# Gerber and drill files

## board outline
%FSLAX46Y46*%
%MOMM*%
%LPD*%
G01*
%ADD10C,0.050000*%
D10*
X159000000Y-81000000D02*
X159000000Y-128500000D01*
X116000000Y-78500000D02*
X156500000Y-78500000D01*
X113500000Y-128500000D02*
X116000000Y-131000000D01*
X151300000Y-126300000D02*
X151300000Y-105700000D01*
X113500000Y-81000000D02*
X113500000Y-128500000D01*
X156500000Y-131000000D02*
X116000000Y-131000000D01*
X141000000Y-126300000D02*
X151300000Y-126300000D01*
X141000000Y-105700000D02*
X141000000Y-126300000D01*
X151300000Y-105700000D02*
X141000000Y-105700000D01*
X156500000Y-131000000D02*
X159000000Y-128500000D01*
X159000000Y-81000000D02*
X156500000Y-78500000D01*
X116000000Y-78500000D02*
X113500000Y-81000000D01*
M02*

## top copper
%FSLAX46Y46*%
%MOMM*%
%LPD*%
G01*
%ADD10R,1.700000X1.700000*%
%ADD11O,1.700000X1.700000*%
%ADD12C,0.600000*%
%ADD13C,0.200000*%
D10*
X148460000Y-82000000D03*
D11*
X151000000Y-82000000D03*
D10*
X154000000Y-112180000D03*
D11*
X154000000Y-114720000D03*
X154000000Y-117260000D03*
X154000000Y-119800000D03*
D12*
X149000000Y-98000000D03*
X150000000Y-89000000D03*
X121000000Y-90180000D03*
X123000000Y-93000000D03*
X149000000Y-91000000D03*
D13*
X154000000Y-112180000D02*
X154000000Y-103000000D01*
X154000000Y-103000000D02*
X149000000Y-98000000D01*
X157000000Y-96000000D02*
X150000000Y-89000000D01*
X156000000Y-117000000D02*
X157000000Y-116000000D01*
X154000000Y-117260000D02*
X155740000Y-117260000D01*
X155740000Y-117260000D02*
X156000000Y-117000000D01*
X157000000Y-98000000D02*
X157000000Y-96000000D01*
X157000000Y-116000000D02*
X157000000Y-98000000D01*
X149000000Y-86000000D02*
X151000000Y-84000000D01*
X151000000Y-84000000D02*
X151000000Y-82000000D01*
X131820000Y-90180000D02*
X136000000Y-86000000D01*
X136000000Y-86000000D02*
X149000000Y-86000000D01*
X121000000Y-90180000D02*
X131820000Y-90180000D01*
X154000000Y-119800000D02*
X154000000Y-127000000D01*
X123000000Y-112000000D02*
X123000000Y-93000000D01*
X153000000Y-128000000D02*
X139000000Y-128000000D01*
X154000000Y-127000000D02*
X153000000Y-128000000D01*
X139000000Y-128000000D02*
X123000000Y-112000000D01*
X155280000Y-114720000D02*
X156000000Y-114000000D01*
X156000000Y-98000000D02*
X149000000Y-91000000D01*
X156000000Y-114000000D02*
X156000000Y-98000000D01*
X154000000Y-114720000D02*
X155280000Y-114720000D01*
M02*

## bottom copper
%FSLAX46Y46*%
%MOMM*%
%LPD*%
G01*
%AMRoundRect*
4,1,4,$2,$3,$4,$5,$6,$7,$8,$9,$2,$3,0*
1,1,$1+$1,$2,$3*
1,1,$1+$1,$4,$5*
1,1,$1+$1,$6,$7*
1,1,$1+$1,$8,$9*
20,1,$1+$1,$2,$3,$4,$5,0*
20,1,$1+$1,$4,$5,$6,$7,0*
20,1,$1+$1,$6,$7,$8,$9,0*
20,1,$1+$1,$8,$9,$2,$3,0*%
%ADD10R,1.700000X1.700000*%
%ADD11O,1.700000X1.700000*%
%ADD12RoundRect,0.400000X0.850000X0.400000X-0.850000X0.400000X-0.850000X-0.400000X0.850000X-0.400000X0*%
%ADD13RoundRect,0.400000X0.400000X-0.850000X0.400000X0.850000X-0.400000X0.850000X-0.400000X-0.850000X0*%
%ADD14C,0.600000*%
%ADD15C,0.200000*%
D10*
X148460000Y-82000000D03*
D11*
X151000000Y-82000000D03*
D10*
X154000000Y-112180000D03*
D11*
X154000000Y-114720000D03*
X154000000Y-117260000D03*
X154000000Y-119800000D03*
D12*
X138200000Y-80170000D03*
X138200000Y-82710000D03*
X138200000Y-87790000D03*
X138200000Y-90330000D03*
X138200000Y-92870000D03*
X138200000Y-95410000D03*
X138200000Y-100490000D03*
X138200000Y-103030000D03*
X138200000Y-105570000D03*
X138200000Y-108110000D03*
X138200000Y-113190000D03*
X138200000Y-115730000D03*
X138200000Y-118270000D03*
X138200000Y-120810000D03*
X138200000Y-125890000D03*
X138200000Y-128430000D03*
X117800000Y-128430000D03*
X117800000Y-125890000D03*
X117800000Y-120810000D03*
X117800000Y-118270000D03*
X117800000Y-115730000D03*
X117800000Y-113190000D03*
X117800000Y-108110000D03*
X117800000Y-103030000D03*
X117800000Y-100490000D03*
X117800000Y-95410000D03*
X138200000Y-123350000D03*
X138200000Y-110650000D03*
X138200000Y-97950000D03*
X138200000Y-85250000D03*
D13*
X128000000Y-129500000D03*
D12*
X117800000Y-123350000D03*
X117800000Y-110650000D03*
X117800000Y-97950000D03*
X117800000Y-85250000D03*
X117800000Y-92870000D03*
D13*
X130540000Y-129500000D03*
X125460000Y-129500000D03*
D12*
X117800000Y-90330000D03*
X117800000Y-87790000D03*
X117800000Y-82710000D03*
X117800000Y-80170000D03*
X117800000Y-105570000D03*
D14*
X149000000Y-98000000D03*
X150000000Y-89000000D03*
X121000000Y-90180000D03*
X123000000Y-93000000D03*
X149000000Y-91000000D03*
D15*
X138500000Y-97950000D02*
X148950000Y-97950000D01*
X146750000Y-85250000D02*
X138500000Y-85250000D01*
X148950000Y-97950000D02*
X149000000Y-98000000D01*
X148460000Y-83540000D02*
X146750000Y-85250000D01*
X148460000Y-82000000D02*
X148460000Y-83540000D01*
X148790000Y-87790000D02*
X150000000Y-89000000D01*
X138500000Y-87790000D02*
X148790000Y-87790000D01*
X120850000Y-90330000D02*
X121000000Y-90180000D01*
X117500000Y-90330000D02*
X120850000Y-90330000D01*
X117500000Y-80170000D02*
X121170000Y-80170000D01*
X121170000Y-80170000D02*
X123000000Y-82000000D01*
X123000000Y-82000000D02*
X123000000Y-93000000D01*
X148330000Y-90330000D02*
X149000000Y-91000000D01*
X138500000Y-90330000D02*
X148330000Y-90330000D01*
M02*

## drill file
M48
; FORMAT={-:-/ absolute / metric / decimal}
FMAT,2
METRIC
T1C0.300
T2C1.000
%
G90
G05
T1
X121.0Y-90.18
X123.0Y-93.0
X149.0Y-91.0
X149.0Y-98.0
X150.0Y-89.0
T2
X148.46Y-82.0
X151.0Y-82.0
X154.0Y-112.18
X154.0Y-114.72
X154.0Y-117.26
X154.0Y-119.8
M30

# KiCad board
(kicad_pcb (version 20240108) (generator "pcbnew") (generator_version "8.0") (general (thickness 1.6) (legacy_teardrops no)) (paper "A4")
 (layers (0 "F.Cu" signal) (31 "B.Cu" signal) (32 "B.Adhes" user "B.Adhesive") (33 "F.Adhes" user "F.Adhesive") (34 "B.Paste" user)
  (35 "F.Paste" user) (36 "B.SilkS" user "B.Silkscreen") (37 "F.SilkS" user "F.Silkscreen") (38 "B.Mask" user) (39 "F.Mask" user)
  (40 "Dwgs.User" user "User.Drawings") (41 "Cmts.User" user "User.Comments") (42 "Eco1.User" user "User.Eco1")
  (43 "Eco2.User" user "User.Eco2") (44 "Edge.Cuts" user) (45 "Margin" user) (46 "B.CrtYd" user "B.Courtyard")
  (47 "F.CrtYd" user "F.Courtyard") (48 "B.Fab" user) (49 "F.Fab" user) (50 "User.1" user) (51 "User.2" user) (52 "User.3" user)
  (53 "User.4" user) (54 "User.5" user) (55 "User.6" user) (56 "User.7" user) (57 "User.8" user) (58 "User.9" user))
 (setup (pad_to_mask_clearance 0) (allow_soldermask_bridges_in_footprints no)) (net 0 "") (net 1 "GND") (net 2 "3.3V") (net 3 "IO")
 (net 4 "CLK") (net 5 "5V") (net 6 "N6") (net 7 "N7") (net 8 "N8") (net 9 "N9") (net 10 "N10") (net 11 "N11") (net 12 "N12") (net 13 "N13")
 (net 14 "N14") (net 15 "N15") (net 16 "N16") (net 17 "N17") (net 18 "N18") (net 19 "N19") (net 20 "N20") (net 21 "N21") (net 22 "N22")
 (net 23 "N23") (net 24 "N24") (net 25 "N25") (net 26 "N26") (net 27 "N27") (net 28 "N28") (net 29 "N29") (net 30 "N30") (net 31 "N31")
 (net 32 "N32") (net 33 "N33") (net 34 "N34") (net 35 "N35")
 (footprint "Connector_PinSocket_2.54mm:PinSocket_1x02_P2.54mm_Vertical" (layer "F.Cu") (at 148.46 82 90)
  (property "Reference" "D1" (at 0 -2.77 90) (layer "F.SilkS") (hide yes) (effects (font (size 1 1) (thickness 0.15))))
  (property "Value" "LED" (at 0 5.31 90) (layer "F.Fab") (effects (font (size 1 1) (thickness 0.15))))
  (pad "1" thru_hole rect (at 0 0 90) (size 1.7 1.7) (drill 1) (layers "*.Cu" "*.Mask") (remove_unused_layers no) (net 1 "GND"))
  (pad "2" thru_hole oval (at 0 2.54 90) (size 1.7 1.7) (drill 1) (layers "*.Cu" "*.Mask") (remove_unused_layers no) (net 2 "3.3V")))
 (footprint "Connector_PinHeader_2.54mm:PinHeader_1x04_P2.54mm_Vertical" (layer "F.Cu") (at 154 112.18)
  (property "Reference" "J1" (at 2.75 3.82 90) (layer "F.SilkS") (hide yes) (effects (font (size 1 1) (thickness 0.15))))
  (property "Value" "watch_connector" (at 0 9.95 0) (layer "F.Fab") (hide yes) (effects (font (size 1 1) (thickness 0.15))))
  (pad "1" thru_hole rect (at 0 0) (size 1.7 1.7) (drill 1) (layers "*.Cu" "*.Mask") (remove_unused_layers no) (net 1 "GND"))
  (pad "2" thru_hole oval (at 0 2.54) (size 1.7 1.7) (drill 1) (layers "*.Cu" "*.Mask") (remove_unused_layers no) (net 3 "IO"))
  (pad "3" thru_hole oval (at 0 5.08) (size 1.7 1.7) (drill 1) (layers "*.Cu" "*.Mask") (remove_unused_layers no) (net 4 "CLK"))
  (pad "4" thru_hole oval (at 0 7.62) (size 1.7 1.7) (drill 1) (layers "*.Cu" "*.Mask") (remove_unused_layers no) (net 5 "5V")))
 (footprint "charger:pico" (layer "B.Cu") (at 128 104.3 180)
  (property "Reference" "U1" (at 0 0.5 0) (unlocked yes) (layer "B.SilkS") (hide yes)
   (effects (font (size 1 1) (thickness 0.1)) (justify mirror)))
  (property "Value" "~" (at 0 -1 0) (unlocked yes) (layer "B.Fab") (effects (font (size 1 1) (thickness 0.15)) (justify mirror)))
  (pad "0" smd roundrect (at -10.5 24.13 180) (size 2.5 1.6) (drill (offset 0.3 0)) (layers "B.Cu" "B.Paste" "B.Mask")
   (roundrect_rratio 0.25) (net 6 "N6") (thermal_bridge_angle 45))
  (pad "1" smd roundrect (at -10.5 21.59 180) (size 2.5 1.6) (drill (offset 0.3 0)) (layers "B.Cu" "B.Paste" "B.Mask")
   (roundrect_rratio 0.25) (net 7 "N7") (thermal_bridge_angle 45))
  (pad "2" smd roundrect (at -10.5 16.51 180) (size 2.5 1.6) (drill (offset 0.3 0)) (layers "B.Cu" "B.Paste" "B.Mask")
   (roundrect_rratio 0.25) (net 4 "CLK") (thermal_bridge_angle 45))
  (pad "3" smd roundrect (at -10.5 13.97 180) (size 2.5 1.6) (drill (offset 0.3 0)) (layers "B.Cu" "B.Paste" "B.Mask")
   (roundrect_rratio 0.25) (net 3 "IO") (thermal_bridge_angle 45))
  (pad "4" smd roundrect (at -10.5 11.43 180) (size 2.5 1.6) (drill (offset 0.3 0)) (layers "B.Cu" "B.Paste" "B.Mask")
   (roundrect_rratio 0.25) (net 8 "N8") (thermal_bridge_angle 45))
  (pad "5" smd roundrect (at -10.5 8.89 180) (size 2.5 1.6) (drill (offset 0.3 0)) (layers "B.Cu" "B.Paste" "B.Mask")
   (roundrect_rratio 0.25) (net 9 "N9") (thermal_bridge_angle 45))
  (pad "6" smd roundrect (at -10.5 3.81 180) (size 2.5 1.6) (drill (offset 0.3 0)) (layers "B.Cu" "B.Paste" "B.Mask")
   (roundrect_rratio 0.25) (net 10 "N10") (thermal_bridge_angle 45))
  (pad "7" smd roundrect (at -10.5 1.27 180) (size 2.5 1.6) (drill (offset 0.3 0)) (layers "B.Cu" "B.Paste" "B.Mask")
   (roundrect_rratio 0.25) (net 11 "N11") (thermal_bridge_angle 45))
  (pad "8" smd roundrect (at -10.5 -1.27 180) (size 2.5 1.6) (drill (offset 0.3 0)) (layers "B.Cu" "B.Paste" "B.Mask")
   (roundrect_rratio 0.25) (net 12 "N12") (thermal_bridge_angle 45))
  (pad "9" smd roundrect (at -10.5 -3.81 180) (size 2.5 1.6) (drill (offset 0.3 0)) (layers "B.Cu" "B.Paste" "B.Mask")
   (roundrect_rratio 0.25) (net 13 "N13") (thermal_bridge_angle 45))
  (pad "10" smd roundrect (at -10.5 -8.89 180) (size 2.5 1.6) (drill (offset 0.3 0)) (layers "B.Cu" "B.Paste" "B.Mask")
   (roundrect_rratio 0.25) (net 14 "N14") (thermal_bridge_angle 45))
  (pad "11" smd roundrect (at -10.5 -11.43 180) (size 2.5 1.6) (drill (offset 0.3 0)) (layers "B.Cu" "B.Paste" "B.Mask")
   (roundrect_rratio 0.25) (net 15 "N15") (thermal_bridge_angle 45))
  (pad "12" smd roundrect (at -10.5 -13.97 180) (size 2.5 1.6) (drill (offset 0.3 0)) (layers "B.Cu" "B.Paste" "B.Mask")
   (roundrect_rratio 0.25) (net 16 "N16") (thermal_bridge_angle 45))
  (pad "13" smd roundrect (at -10.5 -16.51 180) (size 2.5 1.6) (drill (offset 0.3 0)) (layers "B.Cu" "B.Paste" "B.Mask")
   (roundrect_rratio 0.25) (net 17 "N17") (thermal_bridge_angle 45))
  (pad "14" smd roundrect (at -10.5 -21.59 180) (size 2.5 1.6) (drill (offset 0.3 0)) (layers "B.Cu" "B.Paste" "B.Mask")
   (roundrect_rratio 0.25) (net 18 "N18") (thermal_bridge_angle 45))
  (pad "15" smd roundrect (at -10.5 -24.13 180) (size 2.5 1.6) (drill (offset 0.3 0)) (layers "B.Cu" "B.Paste" "B.Mask")
   (roundrect_rratio 0.25) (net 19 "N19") (thermal_bridge_angle 45))
  (pad "16" smd roundrect (at 10.5 -24.13 180) (size 2.5 1.6) (drill (offset -0.3 0)) (layers "B.Cu" "B.Paste" "B.Mask")
   (roundrect_rratio 0.25) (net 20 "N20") (thermal_bridge_angle 45))
  (pad "17" smd roundrect (at 10.5 -21.59 180) (size 2.5 1.6) (drill (offset -0.3 0)) (layers "B.Cu" "B.Paste" "B.Mask")
   (roundrect_rratio 0.25) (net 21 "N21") (thermal_bridge_angle 45))
  (pad "18" smd roundrect (at 10.5 -16.51 180) (size 2.5 1.6) (drill (offset -0.3 0)) (layers "B.Cu" "B.Paste" "B.Mask")
   (roundrect_rratio 0.25) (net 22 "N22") (thermal_bridge_angle 45))
  (pad "19" smd roundrect (at 10.5 -13.97 180) (size 2.5 1.6) (drill (offset -0.3 0)) (layers "B.Cu" "B.Paste" "B.Mask")
   (roundrect_rratio 0.25) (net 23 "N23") (thermal_bridge_angle 45))
  (pad "20" smd roundrect (at 10.5 -11.43 180) (size 2.5 1.6) (drill (offset -0.3 0)) (layers "B.Cu" "B.Paste" "B.Mask")
   (roundrect_rratio 0.25) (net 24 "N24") (thermal_bridge_angle 45))
  (pad "21" smd roundrect (at 10.5 -8.89 180) (size 2.5 1.6) (drill (offset -0.3 0)) (layers "B.Cu" "B.Paste" "B.Mask")
   (roundrect_rratio 0.25) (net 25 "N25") (thermal_bridge_angle 45))
  (pad "22" smd roundrect (at 10.5 -3.81 180) (size 2.5 1.6) (drill (offset -0.3 0)) (layers "B.Cu" "B.Paste" "B.Mask")
   (roundrect_rratio 0.25) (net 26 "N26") (thermal_bridge_angle 45))
  (pad "26" smd roundrect (at 10.5 1.27 180) (size 2.5 1.6) (drill (offset -0.3 0)) (layers "B.Cu" "B.Paste" "B.Mask")
   (roundrect_rratio 0.25) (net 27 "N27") (thermal_bridge_angle 45))
  (pad "27" smd roundrect (at 10.5 3.81 180) (size 2.5 1.6) (drill (offset -0.3 0)) (layers "B.Cu" "B.Paste" "B.Mask")
   (roundrect_rratio 0.25) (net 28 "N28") (thermal_bridge_angle 45))
  (pad "28" smd roundrect (at 10.5 8.89 180) (size 2.5 1.6) (drill (offset -0.3 0)) (layers "B.Cu" "B.Paste" "B.Mask")
   (roundrect_rratio 0.25) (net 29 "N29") (thermal_bridge_angle 45))
  (pad "29" smd roundrect (at -10.5 -19.05 180) (size 2.5 1.6) (drill (offset 0.3 0)) (layers "B.Cu" "B.Paste" "B.Mask")
   (roundrect_rratio 0.25) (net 1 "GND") (thermal_bridge_angle 45))
  (pad "29" smd roundrect (at -10.5 -6.35 180) (size 2.5 1.6) (drill (offset 0.3 0)) (layers "B.Cu" "B.Paste" "B.Mask")
   (roundrect_rratio 0.25) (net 1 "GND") (thermal_bridge_angle 45))
  (pad "29" smd roundrect (at -10.5 6.35 180) (size 2.5 1.6) (drill (offset 0.3 0)) (layers "B.Cu" "B.Paste" "B.Mask")
   (roundrect_rratio 0.25) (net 1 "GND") (thermal_bridge_angle 45))
  (pad "29" smd roundrect (at -10.5 19.05 180) (size 2.5 1.6) (drill (offset 0.3 0)) (layers "B.Cu" "B.Paste" "B.Mask")
   (roundrect_rratio 0.25) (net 1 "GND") (thermal_bridge_angle 45))
  (pad "29" smd roundrect (at 0 -25.5 90) (size 2.5 1.6) (drill (offset 0.3 0)) (layers "B.Cu" "B.Paste" "B.Mask") (roundrect_rratio 0.25)
   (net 1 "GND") (thermal_bridge_angle 45))
  (pad "29" smd roundrect (at 10.5 -19.05 180) (size 2.5 1.6) (drill (offset -0.3 0)) (layers "B.Cu" "B.Paste" "B.Mask")
   (roundrect_rratio 0.25) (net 1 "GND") (thermal_bridge_angle 45))
  (pad "29" smd roundrect (at 10.5 -6.35 180) (size 2.5 1.6) (drill (offset -0.3 0)) (layers "B.Cu" "B.Paste" "B.Mask")
   (roundrect_rratio 0.25) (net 1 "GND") (thermal_bridge_angle 45))
  (pad "29" smd roundrect (at 10.5 6.35 180) (size 2.5 1.6) (drill (offset -0.3 0)) (layers "B.Cu" "B.Paste" "B.Mask")
   (roundrect_rratio 0.25) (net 1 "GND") (thermal_bridge_angle 45))
  (pad "29" smd roundrect (at 10.5 19.05 180) (size 2.5 1.6) (drill (offset -0.3 0)) (layers "B.Cu" "B.Paste" "B.Mask")
   (roundrect_rratio 0.25) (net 1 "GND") (thermal_bridge_angle 45))
  (pad "30" smd roundrect (at 10.5 11.43 180) (size 2.5 1.6) (drill (offset -0.3 0)) (layers "B.Cu" "B.Paste" "B.Mask")
   (roundrect_rratio 0.25) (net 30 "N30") (thermal_bridge_angle 45))
  (pad "31" smd roundrect (at -2.54 -25.5 90) (size 2.5 1.6) (drill (offset 0.3 0)) (layers "B.Cu" "B.Paste" "B.Mask")
   (roundrect_rratio 0.25) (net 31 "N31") (thermal_bridge_angle 45))
  (pad "32" smd roundrect (at 2.54 -25.5 90) (size 2.5 1.6) (drill (offset 0.3 0)) (layers "B.Cu" "B.Paste" "B.Mask")
   (roundrect_rratio 0.25) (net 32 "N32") (thermal_bridge_angle 45))
  (pad "33" smd roundrect (at 10.5 13.97 180) (size 2.5 1.6) (drill (offset -0.3 0)) (layers "B.Cu" "B.Paste" "B.Mask")
   (roundrect_rratio 0.25) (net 2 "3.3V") (thermal_bridge_angle 45))
  (pad "34" smd roundrect (at 10.5 16.51 180) (size 2.5 1.6) (drill (offset -0.3 0)) (layers "B.Cu" "B.Paste" "B.Mask")
   (roundrect_rratio 0.25) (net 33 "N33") (thermal_bridge_angle 45))
  (pad "35" smd roundrect (at 10.5 21.59 180) (size 2.5 1.6) (drill (offset -0.3 0)) (layers "B.Cu" "B.Paste" "B.Mask")
   (roundrect_rratio 0.25) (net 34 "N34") (thermal_bridge_angle 45))
  (pad "36" smd roundrect (at 10.5 24.13 180) (size 2.5 1.6) (drill (offset -0.3 0)) (layers "B.Cu" "B.Paste" "B.Mask")
   (roundrect_rratio 0.25) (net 5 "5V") (thermal_bridge_angle 45))
  (pad "37" smd roundrect (at 10.5 -1.27 180) (size 2.5 1.6) (drill (offset -0.3 0)) (layers "B.Cu" "B.Paste" "B.Mask")
   (roundrect_rratio 0.25) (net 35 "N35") (thermal_bridge_angle 45)))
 (gr_line (start 159 81) (end 159 128.5) (stroke (width 0.05) (type default)) (layer "Edge.Cuts"))
 (gr_line (start 116 78.5) (end 156.5 78.5) (stroke (width 0.05) (type default)) (layer "Edge.Cuts"))
 (gr_line (start 113.5 128.5) (end 116 131) (stroke (width 0.05) (type default)) (layer "Edge.Cuts"))
 (gr_line (start 151.3 126.3) (end 151.3 105.7) (stroke (width 0.05) (type default)) (layer "Edge.Cuts"))
 (gr_line (start 113.5 81) (end 113.5 128.5) (stroke (width 0.05) (type default)) (layer "Edge.Cuts"))
 (gr_line (start 156.5 131) (end 116 131) (stroke (width 0.05) (type default)) (layer "Edge.Cuts"))
 (gr_line (start 141 126.3) (end 151.3 126.3) (stroke (width 0.05) (type default)) (layer "Edge.Cuts"))
 (gr_line (start 141 105.7) (end 141 126.3) (stroke (width 0.05) (type default)) (layer "Edge.Cuts"))
 (gr_line (start 151.3 105.7) (end 141 105.7) (stroke (width 0.05) (type default)) (layer "Edge.Cuts"))
 (gr_line (start 156.5 131) (end 159 128.5) (stroke (width 0.05) (type default)) (layer "Edge.Cuts"))
 (gr_line (start 159 81) (end 156.5 78.5) (stroke (width 0.05) (type default)) (layer "Edge.Cuts"))
 (gr_line (start 116 78.5) (end 113.5 81) (stroke (width 0.05) (type default)) (layer "Edge.Cuts"))
 (segment (start 154 112.18) (end 154 103) (width 0.2) (layer "F.Cu") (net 1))
 (segment (start 154 103) (end 149 98) (width 0.2) (layer "F.Cu") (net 1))
 (via (at 149 98) (size 0.6) (drill 0.3) (layers "F.Cu" "B.Cu") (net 1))
 (segment (start 138.5 97.95) (end 148.95 97.95) (width 0.2) (layer "B.Cu") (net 1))
 (segment (start 146.75 85.25) (end 138.5 85.25) (width 0.2) (layer "B.Cu") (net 1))
 (segment (start 148.95 97.95) (end 149 98) (width 0.2) (layer "B.Cu") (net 1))
 (segment (start 148.46 83.54) (end 146.75 85.25) (width 0.2) (layer "B.Cu") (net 1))
 (segment (start 148.46 82) (end 148.46 83.54) (width 0.2) (layer "B.Cu") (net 1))
 (segment (start 157 96) (end 150 89) (width 0.2) (layer "F.Cu") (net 4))
 (segment (start 156 117) (end 157 116) (width 0.2) (layer "F.Cu") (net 4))
 (segment (start 154 117.26) (end 155.74 117.26) (width 0.2) (layer "F.Cu") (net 4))
 (segment (start 155.74 117.26) (end 156 117) (width 0.2) (layer "F.Cu") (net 4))
 (segment (start 157 98) (end 157 96) (width 0.2) (layer "F.Cu") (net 4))
 (segment (start 157 116) (end 157 98) (width 0.2) (layer "F.Cu") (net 4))
 (via (at 150 89) (size 0.6) (drill 0.3) (layers "F.Cu" "B.Cu") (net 4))
 (segment (start 148.79 87.79) (end 150 89) (width 0.2) (layer "B.Cu") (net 4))
 (segment (start 138.5 87.79) (end 148.79 87.79) (width 0.2) (layer "B.Cu") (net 4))
 (segment (start 149 86) (end 151 84) (width 0.2) (layer "F.Cu") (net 2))
 (segment (start 151 84) (end 151 82) (width 0.2) (layer "F.Cu") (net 2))
 (segment (start 131.82 90.18) (end 136 86) (width 0.2) (layer "F.Cu") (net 2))
 (segment (start 136 86) (end 149 86) (width 0.2) (layer "F.Cu") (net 2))
 (segment (start 121 90.18) (end 131.82 90.18) (width 0.2) (layer "F.Cu") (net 2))
 (via (at 121 90.18) (size 0.6) (drill 0.3) (layers "F.Cu" "B.Cu") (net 2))
 (segment (start 120.85 90.33) (end 121 90.18) (width 0.2) (layer "B.Cu") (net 2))
 (segment (start 117.5 90.33) (end 120.85 90.33) (width 0.2) (layer "B.Cu") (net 2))
 (segment (start 154 119.8) (end 154 127) (width 0.2) (layer "F.Cu") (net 5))
 (segment (start 123 112) (end 123 93) (width 0.2) (layer "F.Cu") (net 5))
 (segment (start 153 128) (end 139 128) (width 0.2) (layer "F.Cu") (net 5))
 (segment (start 154 127) (end 153 128) (width 0.2) (layer "F.Cu") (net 5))
 (segment (start 139 128) (end 123 112) (width 0.2) (layer "F.Cu") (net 5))
 (via (at 123 93) (size 0.6) (drill 0.3) (layers "F.Cu" "B.Cu") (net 5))
 (segment (start 117.5 80.17) (end 121.17 80.17) (width 0.2) (layer "B.Cu") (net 5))
 (segment (start 121.17 80.17) (end 123 82) (width 0.2) (layer "B.Cu") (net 5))
 (segment (start 123 82) (end 123 93) (width 0.2) (layer "B.Cu") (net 5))
 (segment (start 155.28 114.72) (end 156 114) (width 0.2) (layer "F.Cu") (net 3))
 (segment (start 156 98) (end 149 91) (width 0.2) (layer "F.Cu") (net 3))
 (segment (start 156 114) (end 156 98) (width 0.2) (layer "F.Cu") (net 3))
 (segment (start 154 114.72) (end 155.28 114.72) (width 0.2) (layer "F.Cu") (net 3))
 (via (at 149 91) (size 0.6) (drill 0.3) (layers "F.Cu" "B.Cu") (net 3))
 (segment (start 148.33 90.33) (end 149 91) (width 0.2) (layer "B.Cu") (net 3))
 (segment (start 138.5 90.33) (end 148.33 90.33) (width 0.2) (layer "B.Cu") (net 3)))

